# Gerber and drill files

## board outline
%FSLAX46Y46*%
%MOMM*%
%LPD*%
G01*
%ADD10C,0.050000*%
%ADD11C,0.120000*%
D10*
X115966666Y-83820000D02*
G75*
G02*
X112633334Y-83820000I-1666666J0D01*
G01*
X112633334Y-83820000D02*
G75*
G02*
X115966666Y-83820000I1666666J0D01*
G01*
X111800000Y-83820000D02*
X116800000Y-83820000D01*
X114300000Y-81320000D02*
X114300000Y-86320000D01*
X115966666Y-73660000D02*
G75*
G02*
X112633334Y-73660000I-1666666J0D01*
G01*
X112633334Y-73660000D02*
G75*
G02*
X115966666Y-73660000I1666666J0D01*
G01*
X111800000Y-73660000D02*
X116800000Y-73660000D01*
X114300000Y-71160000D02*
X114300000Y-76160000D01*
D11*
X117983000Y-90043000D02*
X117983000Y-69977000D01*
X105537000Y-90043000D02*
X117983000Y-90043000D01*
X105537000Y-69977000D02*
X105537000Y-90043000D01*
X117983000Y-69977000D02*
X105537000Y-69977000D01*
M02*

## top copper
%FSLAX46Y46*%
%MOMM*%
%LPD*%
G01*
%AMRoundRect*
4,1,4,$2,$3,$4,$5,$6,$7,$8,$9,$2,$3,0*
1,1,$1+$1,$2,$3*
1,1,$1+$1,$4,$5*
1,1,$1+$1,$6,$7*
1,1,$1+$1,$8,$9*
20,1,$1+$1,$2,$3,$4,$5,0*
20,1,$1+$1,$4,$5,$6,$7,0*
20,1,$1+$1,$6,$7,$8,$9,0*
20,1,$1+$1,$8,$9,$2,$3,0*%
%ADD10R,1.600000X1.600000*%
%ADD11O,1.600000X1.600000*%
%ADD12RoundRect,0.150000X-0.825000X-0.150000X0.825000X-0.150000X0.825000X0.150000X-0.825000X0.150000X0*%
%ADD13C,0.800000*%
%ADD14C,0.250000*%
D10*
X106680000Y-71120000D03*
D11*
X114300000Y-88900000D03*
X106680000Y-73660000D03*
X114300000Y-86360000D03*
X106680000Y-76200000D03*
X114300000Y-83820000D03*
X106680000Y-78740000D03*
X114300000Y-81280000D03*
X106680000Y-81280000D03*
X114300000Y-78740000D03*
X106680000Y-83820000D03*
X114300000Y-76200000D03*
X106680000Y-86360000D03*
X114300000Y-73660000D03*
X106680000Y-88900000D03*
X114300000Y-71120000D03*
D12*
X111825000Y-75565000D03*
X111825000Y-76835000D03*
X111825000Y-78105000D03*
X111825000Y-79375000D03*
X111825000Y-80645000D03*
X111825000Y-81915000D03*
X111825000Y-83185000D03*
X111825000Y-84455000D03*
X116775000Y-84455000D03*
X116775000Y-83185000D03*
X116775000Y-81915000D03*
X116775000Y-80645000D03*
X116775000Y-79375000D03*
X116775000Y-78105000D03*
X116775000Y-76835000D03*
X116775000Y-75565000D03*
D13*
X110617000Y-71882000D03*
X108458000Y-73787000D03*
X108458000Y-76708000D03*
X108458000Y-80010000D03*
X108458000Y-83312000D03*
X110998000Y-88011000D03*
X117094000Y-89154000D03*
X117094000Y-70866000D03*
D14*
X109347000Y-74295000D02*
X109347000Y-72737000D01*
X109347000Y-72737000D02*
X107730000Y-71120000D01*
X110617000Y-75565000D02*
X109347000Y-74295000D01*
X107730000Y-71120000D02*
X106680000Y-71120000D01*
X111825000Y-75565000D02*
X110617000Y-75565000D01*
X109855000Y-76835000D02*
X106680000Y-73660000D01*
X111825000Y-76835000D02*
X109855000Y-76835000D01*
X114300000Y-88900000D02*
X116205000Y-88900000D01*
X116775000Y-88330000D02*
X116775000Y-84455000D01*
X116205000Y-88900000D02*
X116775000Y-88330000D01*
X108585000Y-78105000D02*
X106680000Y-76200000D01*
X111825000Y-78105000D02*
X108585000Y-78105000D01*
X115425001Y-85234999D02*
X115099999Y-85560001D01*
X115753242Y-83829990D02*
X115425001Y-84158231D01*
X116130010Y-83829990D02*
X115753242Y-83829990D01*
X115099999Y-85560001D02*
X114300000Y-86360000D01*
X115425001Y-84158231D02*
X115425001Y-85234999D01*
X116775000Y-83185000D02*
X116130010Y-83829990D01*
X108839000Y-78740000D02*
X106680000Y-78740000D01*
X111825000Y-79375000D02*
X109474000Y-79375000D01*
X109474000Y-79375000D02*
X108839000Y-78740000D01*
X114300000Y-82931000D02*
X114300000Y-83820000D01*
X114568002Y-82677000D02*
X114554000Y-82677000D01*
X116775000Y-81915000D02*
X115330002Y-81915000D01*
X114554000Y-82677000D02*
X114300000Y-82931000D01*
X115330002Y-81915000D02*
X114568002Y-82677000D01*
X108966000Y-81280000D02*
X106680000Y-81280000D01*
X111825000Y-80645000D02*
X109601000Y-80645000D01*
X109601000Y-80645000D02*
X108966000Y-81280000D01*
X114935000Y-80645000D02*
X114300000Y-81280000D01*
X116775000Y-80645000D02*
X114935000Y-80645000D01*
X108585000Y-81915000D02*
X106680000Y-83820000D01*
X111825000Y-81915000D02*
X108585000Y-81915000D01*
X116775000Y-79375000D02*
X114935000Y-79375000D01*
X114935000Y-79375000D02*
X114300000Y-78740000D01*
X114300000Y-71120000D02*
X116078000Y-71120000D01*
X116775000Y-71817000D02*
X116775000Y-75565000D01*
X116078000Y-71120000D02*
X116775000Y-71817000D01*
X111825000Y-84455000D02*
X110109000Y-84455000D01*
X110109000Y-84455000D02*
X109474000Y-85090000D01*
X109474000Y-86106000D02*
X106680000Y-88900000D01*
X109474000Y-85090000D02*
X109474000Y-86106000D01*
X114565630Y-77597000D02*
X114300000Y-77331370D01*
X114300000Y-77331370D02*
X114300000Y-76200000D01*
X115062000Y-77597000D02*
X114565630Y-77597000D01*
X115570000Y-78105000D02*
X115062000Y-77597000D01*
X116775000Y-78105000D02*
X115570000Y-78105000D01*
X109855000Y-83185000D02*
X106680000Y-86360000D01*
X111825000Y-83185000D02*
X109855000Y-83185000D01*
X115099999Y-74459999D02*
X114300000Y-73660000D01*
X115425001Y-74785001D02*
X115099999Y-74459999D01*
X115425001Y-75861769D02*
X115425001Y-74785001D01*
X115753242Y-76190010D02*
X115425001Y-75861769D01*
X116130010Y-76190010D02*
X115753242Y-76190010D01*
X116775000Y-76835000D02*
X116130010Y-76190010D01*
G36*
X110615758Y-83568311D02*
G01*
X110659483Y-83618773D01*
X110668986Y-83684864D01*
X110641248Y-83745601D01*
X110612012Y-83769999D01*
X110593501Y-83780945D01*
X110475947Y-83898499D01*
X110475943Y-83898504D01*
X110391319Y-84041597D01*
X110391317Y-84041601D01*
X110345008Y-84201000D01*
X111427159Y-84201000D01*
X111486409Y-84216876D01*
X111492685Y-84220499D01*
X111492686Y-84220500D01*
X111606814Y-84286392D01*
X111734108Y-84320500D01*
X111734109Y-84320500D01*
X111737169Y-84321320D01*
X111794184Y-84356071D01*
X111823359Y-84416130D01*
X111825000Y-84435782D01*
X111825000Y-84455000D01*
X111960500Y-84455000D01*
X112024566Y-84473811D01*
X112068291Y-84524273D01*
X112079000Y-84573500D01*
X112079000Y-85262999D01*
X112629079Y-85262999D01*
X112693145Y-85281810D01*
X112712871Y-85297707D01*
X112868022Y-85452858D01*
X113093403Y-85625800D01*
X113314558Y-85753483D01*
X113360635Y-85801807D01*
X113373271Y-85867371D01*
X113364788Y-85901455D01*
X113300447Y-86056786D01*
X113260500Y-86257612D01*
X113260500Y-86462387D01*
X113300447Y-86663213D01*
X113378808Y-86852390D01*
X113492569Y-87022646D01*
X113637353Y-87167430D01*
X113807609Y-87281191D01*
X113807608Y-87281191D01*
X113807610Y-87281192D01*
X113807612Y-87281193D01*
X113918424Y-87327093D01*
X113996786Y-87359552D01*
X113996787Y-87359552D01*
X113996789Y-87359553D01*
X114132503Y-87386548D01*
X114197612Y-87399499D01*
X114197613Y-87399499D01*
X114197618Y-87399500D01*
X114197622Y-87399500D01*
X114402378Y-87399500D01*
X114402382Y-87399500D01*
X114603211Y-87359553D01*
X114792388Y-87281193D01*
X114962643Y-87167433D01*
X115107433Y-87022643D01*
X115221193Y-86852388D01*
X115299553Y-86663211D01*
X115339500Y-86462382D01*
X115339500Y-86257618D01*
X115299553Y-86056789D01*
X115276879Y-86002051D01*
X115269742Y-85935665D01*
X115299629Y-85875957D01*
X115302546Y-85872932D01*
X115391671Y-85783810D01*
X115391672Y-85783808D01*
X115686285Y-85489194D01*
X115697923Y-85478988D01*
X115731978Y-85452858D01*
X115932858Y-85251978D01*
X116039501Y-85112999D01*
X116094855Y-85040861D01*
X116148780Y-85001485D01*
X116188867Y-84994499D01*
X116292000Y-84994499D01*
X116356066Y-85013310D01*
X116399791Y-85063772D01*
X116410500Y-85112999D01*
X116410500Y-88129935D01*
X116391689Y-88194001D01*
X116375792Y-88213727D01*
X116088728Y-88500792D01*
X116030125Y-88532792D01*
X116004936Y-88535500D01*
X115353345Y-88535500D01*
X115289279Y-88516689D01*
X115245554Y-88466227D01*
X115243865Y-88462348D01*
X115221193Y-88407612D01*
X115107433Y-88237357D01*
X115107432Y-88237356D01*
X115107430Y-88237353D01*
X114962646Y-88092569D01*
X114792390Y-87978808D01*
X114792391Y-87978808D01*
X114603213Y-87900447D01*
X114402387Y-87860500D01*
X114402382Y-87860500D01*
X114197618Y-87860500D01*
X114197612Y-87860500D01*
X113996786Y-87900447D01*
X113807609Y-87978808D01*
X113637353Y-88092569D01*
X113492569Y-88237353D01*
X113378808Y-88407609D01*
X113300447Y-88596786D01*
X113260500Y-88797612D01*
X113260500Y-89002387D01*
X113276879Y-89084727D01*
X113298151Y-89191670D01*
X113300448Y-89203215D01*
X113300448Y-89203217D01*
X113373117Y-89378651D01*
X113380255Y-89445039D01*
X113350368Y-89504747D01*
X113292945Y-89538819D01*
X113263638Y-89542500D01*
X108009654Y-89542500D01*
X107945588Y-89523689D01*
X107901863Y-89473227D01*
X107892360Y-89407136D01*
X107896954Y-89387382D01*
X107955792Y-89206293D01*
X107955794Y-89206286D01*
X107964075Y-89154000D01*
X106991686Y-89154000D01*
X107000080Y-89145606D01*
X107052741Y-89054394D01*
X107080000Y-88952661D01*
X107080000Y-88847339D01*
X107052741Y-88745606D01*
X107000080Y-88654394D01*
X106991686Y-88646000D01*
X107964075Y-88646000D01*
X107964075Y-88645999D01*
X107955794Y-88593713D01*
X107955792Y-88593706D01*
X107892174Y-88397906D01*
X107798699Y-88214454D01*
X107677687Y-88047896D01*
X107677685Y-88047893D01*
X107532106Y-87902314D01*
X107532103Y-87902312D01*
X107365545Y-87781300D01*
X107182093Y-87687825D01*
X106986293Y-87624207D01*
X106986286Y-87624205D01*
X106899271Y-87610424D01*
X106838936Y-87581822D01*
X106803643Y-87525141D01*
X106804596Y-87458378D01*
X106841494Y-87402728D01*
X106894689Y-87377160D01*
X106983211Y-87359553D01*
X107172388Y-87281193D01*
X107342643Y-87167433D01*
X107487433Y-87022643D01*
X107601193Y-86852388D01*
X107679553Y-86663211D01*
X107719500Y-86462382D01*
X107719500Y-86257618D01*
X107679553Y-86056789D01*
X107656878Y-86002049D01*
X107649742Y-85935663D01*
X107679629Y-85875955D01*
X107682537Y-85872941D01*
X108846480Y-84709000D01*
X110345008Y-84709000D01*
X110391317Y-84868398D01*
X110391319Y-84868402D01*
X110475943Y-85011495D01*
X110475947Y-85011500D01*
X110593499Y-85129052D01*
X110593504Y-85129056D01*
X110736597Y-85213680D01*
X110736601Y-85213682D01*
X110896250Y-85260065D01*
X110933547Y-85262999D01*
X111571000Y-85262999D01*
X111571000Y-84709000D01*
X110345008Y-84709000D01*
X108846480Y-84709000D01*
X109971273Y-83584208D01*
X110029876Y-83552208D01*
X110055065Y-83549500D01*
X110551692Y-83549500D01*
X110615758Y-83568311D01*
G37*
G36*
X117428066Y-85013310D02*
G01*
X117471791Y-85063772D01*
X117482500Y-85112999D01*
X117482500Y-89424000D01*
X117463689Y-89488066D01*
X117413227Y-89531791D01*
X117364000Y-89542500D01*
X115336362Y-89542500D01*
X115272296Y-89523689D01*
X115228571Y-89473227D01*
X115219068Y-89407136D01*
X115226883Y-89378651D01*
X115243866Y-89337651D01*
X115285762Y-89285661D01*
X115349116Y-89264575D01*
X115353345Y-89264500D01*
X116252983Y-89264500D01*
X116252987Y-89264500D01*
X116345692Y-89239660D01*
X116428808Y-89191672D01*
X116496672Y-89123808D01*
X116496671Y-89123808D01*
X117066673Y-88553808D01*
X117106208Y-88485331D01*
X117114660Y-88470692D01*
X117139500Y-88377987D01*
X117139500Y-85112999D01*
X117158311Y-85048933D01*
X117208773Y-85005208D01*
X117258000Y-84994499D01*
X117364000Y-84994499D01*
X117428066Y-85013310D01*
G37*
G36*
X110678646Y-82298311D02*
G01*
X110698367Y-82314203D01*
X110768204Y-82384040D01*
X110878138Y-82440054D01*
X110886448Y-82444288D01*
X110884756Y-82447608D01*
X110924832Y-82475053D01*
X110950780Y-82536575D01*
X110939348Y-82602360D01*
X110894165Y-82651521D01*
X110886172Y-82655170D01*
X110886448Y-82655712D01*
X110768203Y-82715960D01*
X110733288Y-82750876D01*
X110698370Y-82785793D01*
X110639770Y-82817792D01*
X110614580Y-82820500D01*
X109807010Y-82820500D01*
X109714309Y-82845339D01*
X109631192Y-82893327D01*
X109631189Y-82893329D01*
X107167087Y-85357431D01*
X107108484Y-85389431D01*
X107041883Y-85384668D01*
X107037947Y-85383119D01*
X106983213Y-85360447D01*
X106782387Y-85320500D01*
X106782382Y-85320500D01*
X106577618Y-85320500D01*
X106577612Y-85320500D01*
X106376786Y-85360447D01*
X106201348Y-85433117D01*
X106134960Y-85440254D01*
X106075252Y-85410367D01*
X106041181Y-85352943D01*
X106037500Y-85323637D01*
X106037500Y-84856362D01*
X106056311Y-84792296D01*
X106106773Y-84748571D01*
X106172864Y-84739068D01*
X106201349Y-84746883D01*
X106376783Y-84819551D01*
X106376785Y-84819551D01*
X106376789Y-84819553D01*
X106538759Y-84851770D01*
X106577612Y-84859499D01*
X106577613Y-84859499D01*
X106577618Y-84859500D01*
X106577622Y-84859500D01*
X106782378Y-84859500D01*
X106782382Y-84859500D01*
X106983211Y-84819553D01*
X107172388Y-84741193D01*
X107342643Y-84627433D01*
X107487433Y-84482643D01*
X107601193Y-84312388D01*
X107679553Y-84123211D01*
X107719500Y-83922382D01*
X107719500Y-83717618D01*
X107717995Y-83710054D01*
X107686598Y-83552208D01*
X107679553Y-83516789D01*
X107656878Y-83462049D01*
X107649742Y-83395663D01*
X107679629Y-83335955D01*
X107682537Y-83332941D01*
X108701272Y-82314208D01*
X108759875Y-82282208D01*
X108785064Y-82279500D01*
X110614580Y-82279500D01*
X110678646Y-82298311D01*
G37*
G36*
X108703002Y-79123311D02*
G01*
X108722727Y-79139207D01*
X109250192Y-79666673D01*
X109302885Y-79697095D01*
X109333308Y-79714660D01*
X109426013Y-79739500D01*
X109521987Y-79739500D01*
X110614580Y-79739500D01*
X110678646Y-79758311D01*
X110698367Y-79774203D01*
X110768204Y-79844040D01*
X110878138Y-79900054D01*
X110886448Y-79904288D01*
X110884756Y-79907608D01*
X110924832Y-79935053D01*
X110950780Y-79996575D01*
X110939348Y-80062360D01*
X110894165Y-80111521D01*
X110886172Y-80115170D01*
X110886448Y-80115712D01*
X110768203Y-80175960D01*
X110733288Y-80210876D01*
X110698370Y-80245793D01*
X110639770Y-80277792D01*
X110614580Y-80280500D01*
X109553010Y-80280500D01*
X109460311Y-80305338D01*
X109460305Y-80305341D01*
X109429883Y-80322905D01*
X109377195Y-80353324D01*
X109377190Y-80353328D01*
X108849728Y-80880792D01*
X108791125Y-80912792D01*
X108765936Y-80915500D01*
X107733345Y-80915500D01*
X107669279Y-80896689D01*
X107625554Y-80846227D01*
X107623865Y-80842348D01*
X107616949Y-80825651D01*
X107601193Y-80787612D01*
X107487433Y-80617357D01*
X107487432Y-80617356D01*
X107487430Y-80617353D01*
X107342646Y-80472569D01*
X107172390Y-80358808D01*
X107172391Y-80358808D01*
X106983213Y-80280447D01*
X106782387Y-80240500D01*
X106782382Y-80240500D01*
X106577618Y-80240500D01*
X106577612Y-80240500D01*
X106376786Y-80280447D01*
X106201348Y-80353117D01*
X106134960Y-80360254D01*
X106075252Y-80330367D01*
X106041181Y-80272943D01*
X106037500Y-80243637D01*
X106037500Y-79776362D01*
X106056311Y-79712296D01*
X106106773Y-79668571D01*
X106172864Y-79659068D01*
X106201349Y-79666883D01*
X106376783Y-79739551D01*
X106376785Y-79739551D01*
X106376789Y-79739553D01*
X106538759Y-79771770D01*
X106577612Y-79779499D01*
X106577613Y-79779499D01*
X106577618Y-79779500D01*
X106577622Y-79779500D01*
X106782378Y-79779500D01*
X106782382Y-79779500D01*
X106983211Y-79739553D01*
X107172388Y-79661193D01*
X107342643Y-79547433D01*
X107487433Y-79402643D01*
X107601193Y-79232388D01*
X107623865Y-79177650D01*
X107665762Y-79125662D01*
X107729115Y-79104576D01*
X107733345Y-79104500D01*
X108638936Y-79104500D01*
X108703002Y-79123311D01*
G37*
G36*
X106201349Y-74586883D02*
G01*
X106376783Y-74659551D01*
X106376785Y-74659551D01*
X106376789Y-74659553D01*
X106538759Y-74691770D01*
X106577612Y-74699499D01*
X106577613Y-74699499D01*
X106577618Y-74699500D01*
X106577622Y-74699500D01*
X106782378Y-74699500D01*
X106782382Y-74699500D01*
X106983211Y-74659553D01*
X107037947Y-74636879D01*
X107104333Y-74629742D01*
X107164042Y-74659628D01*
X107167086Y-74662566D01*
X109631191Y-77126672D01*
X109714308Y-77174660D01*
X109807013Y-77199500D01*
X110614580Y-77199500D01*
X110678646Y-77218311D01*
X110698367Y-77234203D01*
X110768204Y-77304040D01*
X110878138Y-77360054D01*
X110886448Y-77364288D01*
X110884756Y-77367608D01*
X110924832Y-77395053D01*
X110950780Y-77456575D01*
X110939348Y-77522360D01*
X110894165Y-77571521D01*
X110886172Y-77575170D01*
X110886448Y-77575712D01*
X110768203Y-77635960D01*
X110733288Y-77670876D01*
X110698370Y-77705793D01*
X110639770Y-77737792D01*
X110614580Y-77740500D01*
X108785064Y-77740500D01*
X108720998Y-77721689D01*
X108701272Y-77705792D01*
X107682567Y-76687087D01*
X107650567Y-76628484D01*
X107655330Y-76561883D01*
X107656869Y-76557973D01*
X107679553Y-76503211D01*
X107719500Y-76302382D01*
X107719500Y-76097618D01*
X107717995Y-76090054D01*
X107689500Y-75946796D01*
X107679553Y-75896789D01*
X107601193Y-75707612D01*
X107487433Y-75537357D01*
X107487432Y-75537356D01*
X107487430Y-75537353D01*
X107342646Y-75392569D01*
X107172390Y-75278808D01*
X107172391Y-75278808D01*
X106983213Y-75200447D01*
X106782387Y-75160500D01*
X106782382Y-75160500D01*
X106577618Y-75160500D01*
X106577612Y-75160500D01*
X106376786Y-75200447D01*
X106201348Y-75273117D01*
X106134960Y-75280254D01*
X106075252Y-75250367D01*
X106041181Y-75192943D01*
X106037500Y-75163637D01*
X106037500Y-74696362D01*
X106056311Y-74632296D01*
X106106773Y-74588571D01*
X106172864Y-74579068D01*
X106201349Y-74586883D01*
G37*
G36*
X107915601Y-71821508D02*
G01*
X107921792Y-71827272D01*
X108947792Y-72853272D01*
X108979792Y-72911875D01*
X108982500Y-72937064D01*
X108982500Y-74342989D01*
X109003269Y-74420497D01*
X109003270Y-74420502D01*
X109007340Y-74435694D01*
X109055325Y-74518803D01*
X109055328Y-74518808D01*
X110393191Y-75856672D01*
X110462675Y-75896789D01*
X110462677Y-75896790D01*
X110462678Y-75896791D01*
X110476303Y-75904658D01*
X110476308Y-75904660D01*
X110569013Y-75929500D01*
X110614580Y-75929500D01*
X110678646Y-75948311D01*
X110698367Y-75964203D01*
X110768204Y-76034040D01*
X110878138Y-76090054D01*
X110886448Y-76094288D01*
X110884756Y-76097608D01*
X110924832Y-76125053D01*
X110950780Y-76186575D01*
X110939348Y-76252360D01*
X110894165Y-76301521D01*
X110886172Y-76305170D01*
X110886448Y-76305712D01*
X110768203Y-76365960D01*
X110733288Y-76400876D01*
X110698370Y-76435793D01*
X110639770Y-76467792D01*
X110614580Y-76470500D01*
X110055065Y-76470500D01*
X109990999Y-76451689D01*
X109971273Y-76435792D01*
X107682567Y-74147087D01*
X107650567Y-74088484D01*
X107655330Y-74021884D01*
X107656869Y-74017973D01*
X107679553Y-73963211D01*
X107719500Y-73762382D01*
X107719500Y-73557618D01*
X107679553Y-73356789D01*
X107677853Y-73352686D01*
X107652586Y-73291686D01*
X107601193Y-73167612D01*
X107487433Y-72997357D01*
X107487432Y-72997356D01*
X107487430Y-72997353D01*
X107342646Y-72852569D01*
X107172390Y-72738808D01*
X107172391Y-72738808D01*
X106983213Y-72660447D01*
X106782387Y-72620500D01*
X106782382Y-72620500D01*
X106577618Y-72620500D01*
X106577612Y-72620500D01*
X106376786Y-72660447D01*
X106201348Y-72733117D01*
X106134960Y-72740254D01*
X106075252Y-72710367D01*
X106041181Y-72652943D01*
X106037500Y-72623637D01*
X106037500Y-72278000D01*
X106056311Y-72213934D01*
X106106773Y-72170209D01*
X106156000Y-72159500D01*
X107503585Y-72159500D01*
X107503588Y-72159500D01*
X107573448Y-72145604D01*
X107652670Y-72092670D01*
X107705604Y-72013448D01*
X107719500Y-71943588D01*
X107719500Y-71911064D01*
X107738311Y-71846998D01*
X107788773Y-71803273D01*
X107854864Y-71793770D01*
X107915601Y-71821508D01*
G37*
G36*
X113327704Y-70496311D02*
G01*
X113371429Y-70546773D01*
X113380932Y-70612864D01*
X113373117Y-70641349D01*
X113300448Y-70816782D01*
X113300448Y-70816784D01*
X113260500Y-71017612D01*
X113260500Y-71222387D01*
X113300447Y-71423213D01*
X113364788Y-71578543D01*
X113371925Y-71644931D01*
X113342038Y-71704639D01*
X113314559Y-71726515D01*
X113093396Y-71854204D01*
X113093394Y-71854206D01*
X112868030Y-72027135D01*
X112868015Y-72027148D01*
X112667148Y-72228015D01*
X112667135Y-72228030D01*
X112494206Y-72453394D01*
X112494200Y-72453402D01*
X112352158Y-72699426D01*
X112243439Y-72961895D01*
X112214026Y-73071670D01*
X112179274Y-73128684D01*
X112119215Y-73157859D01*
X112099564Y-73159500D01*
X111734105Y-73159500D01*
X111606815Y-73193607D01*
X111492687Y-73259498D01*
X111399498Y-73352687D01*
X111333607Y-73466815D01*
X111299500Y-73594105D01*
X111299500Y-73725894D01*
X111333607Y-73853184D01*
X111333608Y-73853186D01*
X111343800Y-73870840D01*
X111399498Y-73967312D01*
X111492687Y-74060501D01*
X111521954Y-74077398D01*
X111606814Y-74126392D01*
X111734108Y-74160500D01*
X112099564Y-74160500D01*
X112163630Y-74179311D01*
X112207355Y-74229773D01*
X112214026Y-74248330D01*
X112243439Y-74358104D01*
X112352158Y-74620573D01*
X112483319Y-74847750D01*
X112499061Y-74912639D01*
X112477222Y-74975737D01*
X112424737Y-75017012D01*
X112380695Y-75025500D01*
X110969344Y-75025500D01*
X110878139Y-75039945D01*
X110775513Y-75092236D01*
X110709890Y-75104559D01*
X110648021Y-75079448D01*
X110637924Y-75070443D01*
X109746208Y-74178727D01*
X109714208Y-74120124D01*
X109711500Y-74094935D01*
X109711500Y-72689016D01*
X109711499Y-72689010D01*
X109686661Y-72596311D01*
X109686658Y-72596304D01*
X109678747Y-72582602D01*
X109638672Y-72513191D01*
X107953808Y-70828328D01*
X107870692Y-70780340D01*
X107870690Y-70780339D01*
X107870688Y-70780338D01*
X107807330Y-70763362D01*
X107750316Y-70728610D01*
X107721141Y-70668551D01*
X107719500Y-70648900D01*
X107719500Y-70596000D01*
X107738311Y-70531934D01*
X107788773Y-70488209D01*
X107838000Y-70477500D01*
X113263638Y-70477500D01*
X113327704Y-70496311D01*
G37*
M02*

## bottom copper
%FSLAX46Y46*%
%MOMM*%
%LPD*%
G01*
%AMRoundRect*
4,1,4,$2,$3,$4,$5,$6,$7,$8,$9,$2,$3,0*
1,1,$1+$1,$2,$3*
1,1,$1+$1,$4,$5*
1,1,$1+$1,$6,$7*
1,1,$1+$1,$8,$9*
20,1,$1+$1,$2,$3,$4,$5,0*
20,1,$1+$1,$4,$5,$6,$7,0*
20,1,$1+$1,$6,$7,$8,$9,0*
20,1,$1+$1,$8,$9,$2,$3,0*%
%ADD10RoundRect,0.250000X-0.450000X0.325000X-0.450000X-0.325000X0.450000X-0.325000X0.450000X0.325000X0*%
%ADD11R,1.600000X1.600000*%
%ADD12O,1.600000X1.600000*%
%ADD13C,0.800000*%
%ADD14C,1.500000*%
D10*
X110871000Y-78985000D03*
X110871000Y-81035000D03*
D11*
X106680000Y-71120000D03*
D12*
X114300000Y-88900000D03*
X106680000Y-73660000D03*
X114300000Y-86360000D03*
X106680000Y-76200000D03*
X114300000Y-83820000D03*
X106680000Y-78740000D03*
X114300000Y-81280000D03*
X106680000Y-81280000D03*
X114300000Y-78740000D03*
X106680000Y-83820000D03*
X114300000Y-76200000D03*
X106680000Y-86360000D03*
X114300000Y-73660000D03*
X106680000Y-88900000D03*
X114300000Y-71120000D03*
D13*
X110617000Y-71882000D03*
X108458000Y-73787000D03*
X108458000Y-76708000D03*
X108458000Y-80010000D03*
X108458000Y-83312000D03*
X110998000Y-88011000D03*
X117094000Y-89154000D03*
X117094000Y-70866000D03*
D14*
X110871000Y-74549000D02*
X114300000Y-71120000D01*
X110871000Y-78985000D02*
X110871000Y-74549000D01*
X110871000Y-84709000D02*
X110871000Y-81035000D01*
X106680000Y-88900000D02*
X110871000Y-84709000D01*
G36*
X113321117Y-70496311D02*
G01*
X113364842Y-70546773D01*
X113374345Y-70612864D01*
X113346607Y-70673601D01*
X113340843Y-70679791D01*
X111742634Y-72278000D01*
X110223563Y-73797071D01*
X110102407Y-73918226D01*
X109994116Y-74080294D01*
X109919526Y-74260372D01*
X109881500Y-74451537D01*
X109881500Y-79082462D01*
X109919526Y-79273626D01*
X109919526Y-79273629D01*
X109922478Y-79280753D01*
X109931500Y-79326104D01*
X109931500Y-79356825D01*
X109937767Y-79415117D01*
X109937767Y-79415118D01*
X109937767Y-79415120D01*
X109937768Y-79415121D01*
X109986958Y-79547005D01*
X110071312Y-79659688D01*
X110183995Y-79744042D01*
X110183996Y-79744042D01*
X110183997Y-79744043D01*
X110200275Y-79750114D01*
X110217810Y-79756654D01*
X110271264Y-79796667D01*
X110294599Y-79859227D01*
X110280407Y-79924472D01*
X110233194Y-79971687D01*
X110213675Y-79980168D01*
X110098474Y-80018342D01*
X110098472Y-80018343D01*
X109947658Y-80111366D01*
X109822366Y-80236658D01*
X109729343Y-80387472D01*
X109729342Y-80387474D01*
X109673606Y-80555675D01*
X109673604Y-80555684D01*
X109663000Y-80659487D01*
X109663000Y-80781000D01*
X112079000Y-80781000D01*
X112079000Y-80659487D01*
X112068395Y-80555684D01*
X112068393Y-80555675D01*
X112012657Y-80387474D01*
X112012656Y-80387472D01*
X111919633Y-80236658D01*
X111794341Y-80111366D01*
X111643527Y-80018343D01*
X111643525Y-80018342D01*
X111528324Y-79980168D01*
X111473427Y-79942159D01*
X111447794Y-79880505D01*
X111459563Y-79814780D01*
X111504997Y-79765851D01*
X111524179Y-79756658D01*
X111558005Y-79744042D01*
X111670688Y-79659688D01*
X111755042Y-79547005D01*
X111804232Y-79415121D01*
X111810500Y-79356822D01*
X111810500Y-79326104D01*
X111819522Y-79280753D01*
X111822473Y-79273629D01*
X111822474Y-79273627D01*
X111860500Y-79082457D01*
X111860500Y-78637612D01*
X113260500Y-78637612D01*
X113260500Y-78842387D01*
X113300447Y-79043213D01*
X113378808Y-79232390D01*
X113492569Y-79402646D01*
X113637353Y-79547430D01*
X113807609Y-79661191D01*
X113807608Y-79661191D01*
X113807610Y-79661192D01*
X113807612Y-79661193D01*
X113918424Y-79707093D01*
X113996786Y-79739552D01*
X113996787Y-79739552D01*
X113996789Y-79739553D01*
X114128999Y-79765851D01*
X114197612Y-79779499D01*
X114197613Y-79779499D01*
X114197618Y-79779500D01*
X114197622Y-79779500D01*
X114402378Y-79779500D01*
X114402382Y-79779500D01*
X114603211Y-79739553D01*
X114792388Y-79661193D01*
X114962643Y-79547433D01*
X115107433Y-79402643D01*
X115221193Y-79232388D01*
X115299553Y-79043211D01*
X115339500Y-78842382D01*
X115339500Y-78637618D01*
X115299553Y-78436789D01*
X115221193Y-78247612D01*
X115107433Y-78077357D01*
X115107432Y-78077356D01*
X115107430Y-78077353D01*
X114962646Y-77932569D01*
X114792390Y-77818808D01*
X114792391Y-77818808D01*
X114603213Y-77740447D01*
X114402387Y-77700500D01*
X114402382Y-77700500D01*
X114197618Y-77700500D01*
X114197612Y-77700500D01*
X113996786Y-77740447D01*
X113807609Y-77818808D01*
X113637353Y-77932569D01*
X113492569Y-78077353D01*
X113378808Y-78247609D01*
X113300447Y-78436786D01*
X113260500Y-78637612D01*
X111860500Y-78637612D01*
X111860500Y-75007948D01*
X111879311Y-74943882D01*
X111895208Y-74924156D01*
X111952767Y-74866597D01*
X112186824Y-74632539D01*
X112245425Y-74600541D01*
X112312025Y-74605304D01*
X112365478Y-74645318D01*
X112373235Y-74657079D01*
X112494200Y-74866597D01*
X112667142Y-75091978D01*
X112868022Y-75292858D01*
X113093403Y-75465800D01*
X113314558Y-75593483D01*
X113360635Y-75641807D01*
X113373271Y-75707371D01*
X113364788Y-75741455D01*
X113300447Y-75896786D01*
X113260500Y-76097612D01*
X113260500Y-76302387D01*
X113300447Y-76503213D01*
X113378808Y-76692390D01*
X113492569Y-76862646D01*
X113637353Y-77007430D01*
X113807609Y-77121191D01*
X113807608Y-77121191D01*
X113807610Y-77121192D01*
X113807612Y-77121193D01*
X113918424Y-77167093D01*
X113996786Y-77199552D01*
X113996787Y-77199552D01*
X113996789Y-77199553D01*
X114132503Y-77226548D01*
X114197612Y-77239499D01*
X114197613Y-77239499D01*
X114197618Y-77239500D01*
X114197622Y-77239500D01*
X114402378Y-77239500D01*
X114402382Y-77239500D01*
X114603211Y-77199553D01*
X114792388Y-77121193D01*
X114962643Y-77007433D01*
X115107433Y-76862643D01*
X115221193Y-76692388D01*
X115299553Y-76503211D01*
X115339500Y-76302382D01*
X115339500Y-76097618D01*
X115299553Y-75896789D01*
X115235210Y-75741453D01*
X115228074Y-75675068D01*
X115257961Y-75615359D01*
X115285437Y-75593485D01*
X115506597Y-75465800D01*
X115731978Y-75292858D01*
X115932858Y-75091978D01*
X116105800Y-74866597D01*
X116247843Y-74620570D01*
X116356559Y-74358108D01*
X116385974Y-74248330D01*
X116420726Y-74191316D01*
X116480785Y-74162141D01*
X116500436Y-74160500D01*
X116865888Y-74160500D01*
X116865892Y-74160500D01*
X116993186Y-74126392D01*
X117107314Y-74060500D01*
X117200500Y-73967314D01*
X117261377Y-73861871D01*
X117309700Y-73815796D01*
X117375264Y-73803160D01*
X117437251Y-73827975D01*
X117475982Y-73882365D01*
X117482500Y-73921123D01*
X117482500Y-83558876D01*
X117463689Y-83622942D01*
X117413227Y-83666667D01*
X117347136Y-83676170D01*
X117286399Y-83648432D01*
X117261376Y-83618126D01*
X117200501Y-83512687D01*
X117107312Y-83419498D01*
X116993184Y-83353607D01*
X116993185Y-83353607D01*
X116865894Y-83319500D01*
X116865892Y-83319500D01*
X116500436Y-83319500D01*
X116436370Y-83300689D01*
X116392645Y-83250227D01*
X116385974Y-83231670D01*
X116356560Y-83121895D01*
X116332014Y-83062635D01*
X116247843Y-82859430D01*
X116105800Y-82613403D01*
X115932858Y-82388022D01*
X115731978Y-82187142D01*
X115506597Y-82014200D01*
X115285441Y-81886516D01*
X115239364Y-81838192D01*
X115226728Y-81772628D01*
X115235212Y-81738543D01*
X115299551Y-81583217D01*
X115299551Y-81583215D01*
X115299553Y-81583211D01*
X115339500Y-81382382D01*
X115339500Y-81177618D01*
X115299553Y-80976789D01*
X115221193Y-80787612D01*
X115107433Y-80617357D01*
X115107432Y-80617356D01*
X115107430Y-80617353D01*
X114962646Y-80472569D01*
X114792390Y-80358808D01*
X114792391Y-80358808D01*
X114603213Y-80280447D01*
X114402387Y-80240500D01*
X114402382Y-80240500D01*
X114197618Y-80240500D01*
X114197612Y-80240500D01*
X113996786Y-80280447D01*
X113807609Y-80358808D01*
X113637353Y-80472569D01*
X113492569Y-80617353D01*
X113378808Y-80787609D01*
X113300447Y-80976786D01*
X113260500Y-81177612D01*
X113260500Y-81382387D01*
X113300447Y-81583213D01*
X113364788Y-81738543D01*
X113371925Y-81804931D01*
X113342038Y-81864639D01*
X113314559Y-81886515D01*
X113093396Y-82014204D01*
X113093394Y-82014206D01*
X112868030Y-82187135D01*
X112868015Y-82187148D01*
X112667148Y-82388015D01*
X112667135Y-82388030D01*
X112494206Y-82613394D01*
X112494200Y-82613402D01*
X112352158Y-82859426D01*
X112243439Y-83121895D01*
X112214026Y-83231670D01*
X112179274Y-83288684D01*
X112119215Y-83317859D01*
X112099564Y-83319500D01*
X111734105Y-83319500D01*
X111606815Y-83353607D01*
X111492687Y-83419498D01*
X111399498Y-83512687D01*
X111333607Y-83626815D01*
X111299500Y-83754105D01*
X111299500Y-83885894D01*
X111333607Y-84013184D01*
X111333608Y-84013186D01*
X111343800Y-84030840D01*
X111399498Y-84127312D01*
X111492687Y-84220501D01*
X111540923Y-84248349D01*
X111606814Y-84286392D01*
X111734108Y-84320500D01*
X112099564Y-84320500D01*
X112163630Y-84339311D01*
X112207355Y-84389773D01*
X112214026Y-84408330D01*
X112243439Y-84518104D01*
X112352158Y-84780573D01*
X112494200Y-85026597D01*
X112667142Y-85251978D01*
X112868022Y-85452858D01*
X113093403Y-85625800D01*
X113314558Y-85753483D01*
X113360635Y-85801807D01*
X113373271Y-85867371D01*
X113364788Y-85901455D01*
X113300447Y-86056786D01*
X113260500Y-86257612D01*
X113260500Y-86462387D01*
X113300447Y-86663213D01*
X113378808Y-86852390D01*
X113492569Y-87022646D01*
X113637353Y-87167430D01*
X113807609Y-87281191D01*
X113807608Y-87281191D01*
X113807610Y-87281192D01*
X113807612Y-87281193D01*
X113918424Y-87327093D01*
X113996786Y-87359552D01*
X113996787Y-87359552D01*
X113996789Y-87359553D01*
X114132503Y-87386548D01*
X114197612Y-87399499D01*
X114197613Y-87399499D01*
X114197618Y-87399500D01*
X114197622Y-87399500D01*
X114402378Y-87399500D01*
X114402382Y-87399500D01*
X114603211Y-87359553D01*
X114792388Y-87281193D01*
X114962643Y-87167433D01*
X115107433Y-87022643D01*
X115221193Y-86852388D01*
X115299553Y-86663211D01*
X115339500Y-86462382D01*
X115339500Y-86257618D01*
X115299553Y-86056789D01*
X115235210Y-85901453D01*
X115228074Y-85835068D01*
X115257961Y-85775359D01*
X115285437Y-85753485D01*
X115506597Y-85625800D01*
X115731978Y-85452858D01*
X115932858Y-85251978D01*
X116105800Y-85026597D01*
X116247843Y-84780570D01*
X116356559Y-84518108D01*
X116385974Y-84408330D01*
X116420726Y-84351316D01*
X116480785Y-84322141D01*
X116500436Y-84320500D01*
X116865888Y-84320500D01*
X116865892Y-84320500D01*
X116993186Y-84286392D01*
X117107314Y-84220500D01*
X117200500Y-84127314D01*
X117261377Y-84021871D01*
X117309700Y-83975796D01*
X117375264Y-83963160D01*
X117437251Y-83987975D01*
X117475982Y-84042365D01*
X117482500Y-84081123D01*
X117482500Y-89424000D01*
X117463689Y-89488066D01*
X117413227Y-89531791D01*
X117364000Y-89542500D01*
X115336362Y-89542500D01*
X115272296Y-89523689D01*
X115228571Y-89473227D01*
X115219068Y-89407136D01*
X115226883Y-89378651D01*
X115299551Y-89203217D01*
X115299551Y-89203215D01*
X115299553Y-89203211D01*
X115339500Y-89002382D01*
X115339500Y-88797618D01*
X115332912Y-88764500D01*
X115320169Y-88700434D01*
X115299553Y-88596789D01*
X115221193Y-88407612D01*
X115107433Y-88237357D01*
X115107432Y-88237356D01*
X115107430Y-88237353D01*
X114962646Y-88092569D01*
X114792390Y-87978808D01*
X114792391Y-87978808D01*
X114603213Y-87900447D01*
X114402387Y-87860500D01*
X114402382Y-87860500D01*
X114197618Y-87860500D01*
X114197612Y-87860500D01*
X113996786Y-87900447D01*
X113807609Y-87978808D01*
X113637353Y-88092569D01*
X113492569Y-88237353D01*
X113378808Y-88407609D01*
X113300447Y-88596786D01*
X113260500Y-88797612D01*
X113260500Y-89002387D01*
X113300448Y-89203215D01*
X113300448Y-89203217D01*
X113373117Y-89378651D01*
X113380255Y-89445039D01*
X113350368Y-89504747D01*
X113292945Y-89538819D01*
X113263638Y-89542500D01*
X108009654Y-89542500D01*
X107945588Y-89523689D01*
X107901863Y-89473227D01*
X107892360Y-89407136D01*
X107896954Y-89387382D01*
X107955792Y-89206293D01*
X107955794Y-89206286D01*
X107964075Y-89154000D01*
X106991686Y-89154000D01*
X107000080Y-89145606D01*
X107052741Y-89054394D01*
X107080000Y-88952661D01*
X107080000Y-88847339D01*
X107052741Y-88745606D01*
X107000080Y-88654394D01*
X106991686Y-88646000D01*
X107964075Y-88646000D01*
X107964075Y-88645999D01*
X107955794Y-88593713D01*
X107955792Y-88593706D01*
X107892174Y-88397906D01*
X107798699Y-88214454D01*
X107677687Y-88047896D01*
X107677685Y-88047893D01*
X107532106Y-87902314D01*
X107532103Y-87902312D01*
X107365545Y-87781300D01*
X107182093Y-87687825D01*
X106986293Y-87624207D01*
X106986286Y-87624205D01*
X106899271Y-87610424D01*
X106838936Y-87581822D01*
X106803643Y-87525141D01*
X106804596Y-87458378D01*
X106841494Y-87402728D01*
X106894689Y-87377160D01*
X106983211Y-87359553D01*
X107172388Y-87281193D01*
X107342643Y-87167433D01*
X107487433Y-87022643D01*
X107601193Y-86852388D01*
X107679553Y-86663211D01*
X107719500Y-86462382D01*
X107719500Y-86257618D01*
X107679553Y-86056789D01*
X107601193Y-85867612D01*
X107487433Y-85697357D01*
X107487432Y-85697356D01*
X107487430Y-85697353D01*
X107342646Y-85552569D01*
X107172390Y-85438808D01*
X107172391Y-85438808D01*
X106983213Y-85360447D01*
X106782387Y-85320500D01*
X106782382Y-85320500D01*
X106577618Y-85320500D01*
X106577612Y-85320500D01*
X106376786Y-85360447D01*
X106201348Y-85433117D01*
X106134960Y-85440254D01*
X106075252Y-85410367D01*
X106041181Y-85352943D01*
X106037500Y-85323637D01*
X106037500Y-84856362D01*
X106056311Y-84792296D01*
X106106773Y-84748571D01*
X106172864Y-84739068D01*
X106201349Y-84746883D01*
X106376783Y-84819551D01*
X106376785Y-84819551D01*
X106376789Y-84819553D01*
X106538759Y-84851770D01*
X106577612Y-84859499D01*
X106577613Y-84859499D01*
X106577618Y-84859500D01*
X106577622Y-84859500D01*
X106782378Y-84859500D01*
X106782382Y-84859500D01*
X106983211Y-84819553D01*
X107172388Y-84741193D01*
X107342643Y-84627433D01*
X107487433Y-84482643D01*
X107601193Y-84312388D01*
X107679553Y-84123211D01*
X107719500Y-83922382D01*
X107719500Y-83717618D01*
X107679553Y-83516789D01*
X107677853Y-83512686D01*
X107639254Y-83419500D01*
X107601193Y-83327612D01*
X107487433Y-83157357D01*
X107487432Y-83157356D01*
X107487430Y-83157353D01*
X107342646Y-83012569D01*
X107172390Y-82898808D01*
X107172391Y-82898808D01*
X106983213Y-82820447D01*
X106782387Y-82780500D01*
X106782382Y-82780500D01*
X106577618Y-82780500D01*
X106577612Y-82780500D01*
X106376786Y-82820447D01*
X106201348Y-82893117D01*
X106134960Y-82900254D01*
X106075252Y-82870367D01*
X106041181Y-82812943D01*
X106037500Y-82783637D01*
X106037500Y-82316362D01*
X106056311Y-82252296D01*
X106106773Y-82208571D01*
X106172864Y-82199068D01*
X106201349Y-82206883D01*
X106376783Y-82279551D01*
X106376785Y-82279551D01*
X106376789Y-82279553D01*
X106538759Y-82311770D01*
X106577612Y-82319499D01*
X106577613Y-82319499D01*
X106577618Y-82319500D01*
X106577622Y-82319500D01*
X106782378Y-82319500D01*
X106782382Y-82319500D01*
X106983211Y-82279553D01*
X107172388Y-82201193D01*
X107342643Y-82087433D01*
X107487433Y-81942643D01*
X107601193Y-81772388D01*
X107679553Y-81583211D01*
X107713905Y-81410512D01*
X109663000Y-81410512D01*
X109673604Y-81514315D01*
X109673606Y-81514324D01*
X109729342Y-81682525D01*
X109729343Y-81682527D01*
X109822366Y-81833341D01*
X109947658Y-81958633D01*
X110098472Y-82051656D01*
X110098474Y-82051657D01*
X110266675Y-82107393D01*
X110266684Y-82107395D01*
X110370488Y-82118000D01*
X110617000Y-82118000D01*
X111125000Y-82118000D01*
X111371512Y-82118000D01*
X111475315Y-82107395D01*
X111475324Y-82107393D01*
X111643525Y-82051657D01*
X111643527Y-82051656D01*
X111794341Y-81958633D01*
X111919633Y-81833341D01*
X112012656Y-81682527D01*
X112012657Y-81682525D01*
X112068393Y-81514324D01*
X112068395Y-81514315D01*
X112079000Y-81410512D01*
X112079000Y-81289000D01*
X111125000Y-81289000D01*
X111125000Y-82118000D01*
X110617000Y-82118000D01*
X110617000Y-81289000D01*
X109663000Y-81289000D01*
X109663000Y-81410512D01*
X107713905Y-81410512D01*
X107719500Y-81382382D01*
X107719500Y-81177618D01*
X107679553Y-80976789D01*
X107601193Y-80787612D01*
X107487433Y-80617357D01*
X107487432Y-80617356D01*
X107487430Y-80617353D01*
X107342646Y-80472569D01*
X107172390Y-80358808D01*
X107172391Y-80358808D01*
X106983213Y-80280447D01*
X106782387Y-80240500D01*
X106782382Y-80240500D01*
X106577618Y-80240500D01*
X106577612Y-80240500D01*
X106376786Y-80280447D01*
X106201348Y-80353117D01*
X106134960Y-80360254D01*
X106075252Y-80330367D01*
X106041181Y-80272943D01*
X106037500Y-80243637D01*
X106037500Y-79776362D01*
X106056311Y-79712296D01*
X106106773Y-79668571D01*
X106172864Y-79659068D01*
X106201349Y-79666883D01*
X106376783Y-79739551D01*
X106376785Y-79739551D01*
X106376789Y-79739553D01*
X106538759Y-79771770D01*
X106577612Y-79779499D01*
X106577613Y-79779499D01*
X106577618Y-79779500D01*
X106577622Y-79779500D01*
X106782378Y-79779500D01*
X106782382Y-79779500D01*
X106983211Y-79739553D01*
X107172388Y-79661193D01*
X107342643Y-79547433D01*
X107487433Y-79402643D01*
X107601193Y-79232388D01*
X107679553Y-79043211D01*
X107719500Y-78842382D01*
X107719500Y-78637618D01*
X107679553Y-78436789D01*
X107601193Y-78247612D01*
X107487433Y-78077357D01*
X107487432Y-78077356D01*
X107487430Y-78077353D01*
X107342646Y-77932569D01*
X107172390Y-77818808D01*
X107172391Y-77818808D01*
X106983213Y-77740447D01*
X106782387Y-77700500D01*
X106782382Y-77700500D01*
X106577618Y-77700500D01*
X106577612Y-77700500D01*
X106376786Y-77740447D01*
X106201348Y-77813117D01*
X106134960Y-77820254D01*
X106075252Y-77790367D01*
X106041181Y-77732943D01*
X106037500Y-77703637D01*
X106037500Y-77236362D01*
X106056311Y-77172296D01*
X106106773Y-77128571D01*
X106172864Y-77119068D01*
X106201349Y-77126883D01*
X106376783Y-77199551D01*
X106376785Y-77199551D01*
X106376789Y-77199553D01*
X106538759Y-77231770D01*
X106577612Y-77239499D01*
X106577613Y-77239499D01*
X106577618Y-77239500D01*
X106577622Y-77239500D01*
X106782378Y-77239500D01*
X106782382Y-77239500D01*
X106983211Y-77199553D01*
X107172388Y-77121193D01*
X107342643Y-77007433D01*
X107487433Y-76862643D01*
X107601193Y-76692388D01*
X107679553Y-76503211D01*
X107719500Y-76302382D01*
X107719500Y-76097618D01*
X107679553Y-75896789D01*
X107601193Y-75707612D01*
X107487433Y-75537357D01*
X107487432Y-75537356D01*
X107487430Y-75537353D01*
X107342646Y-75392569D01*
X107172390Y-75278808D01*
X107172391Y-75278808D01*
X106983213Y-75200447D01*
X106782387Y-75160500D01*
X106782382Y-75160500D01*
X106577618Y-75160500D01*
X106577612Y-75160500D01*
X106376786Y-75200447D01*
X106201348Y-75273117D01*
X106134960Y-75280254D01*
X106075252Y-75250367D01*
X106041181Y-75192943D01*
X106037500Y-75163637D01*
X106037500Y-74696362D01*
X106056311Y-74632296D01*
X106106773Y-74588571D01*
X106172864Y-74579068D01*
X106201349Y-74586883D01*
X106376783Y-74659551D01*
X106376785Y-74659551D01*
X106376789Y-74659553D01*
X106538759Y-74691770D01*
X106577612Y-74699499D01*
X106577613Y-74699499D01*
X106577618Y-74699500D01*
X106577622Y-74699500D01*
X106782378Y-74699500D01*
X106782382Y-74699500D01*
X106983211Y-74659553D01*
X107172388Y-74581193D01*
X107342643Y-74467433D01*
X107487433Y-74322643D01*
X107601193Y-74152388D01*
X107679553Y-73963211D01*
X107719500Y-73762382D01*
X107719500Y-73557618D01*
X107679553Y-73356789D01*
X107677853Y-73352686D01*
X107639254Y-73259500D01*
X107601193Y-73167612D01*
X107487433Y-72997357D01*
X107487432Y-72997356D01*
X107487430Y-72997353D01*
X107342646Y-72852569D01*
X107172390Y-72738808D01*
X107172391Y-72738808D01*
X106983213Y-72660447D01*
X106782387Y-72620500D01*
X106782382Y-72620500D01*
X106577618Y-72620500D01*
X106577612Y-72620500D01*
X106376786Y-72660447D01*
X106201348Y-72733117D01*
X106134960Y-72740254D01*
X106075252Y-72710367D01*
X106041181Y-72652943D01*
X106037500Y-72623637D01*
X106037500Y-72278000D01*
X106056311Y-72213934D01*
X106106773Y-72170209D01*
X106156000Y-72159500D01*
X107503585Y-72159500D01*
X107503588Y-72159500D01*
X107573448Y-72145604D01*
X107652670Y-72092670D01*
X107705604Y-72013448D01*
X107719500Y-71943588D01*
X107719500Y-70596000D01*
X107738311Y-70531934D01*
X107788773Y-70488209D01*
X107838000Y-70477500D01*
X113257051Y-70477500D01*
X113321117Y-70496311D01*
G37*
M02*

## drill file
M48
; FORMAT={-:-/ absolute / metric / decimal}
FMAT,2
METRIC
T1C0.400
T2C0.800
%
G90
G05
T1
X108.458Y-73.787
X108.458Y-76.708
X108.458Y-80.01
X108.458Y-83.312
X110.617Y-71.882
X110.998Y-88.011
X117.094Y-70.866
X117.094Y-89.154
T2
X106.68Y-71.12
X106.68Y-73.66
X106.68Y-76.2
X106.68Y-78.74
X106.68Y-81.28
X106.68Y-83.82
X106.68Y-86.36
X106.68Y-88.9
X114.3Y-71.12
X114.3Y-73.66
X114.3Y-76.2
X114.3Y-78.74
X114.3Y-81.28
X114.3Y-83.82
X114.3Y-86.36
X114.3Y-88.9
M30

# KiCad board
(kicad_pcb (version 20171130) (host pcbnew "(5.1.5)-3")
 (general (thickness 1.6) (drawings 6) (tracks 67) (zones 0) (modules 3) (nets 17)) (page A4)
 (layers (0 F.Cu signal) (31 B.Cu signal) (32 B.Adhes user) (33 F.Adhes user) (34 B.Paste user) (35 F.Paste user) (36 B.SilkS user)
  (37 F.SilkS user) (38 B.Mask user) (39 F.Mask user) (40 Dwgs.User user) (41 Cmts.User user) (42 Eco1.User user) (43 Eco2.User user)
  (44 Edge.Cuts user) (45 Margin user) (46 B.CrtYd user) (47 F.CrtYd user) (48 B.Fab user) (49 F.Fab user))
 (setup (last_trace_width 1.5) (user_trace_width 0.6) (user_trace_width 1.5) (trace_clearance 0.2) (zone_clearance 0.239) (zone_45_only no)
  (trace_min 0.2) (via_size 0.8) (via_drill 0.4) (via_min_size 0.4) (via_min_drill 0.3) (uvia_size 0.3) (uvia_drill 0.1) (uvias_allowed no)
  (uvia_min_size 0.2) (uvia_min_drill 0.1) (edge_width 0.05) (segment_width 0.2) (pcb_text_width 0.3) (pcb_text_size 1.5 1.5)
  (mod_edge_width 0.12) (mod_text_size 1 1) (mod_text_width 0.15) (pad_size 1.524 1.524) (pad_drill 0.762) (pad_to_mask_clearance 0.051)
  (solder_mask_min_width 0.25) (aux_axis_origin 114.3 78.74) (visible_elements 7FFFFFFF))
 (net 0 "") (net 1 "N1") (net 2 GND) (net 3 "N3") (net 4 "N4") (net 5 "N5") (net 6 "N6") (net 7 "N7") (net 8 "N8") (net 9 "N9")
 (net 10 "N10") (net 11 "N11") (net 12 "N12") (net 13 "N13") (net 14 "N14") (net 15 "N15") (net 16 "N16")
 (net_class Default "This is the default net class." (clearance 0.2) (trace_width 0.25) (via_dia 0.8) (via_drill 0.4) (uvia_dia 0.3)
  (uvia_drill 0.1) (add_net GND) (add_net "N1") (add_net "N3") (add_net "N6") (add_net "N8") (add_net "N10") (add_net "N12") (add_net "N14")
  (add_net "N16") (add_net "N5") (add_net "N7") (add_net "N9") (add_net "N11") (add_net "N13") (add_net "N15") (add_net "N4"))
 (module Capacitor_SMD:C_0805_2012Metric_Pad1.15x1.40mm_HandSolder (layer B.Cu) (at 110.871 80.01 270)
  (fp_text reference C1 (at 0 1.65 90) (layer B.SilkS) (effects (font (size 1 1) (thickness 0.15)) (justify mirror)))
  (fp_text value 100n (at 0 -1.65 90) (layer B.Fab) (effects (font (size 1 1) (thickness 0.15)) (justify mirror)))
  (pad 1 smd roundrect (at -1.025 0 270) (size 1.15 1.4) (layers B.Cu B.Paste B.Mask) (roundrect_rratio 0.217391) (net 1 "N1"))
  (pad 2 smd roundrect (at 1.025 0 270) (size 1.15 1.4) (layers B.Cu B.Paste B.Mask) (roundrect_rratio 0.217391) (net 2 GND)))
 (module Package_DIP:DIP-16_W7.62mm (layer F.Cu) (at 106.68 71.12)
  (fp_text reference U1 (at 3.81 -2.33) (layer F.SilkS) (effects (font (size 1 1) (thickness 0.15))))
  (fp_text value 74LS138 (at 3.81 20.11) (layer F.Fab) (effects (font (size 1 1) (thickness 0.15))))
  (pad 1 thru_hole rect (at 0 0) (size 1.6 1.6) (drill 0.8) (layers *.Cu *.Mask) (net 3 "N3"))
  (pad 9 thru_hole oval (at 7.62 17.78) (size 1.6 1.6) (drill 0.8) (layers *.Cu *.Mask) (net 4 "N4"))
  (pad 2 thru_hole oval (at 0 2.54) (size 1.6 1.6) (drill 0.8) (layers *.Cu *.Mask) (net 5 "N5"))
  (pad 10 thru_hole oval (at 7.62 15.24) (size 1.6 1.6) (drill 0.8) (layers *.Cu *.Mask) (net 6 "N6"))
  (pad 3 thru_hole oval (at 0 5.08) (size 1.6 1.6) (drill 0.8) (layers *.Cu *.Mask) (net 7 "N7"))
  (pad 11 thru_hole oval (at 7.62 12.7) (size 1.6 1.6) (drill 0.8) (layers *.Cu *.Mask) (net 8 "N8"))
  (pad 4 thru_hole oval (at 0 7.62) (size 1.6 1.6) (drill 0.8) (layers *.Cu *.Mask) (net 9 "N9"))
  (pad 12 thru_hole oval (at 7.62 10.16) (size 1.6 1.6) (drill 0.8) (layers *.Cu *.Mask) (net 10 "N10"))
  (pad 5 thru_hole oval (at 0 10.16) (size 1.6 1.6) (drill 0.8) (layers *.Cu *.Mask) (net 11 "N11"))
  (pad 13 thru_hole oval (at 7.62 7.62) (size 1.6 1.6) (drill 0.8) (layers *.Cu *.Mask) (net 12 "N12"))
  (pad 6 thru_hole oval (at 0 12.7) (size 1.6 1.6) (drill 0.8) (layers *.Cu *.Mask) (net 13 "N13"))
  (pad 14 thru_hole oval (at 7.62 5.08) (size 1.6 1.6) (drill 0.8) (layers *.Cu *.Mask) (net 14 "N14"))
  (pad 7 thru_hole oval (at 0 15.24) (size 1.6 1.6) (drill 0.8) (layers *.Cu *.Mask) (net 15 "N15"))
  (pad 15 thru_hole oval (at 7.62 2.54) (size 1.6 1.6) (drill 0.8) (layers *.Cu *.Mask) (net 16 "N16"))
  (pad 8 thru_hole oval (at 0 17.78) (size 1.6 1.6) (drill 0.8) (layers *.Cu *.Mask) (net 2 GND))
  (pad 16 thru_hole oval (at 7.62 0) (size 1.6 1.6) (drill 0.8) (layers *.Cu *.Mask) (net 1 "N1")))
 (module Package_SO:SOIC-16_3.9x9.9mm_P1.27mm (layer F.Cu) (at 114.3 80.01)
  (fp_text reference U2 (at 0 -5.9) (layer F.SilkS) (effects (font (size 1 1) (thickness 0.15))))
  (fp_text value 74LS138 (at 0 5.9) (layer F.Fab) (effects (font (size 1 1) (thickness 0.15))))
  (pad 1 smd roundrect (at -2.475 -4.445) (size 1.95 0.6) (layers F.Cu F.Paste F.Mask) (roundrect_rratio 0.25) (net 3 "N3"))
  (pad 2 smd roundrect (at -2.475 -3.175) (size 1.95 0.6) (layers F.Cu F.Paste F.Mask) (roundrect_rratio 0.25) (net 5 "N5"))
  (pad 3 smd roundrect (at -2.475 -1.905) (size 1.95 0.6) (layers F.Cu F.Paste F.Mask) (roundrect_rratio 0.25) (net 7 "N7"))
  (pad 4 smd roundrect (at -2.475 -0.635) (size 1.95 0.6) (layers F.Cu F.Paste F.Mask) (roundrect_rratio 0.25) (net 9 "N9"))
  (pad 5 smd roundrect (at -2.475 0.635) (size 1.95 0.6) (layers F.Cu F.Paste F.Mask) (roundrect_rratio 0.25) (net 11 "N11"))
  (pad 6 smd roundrect (at -2.475 1.905) (size 1.95 0.6) (layers F.Cu F.Paste F.Mask) (roundrect_rratio 0.25) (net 13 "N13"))
  (pad 7 smd roundrect (at -2.475 3.175) (size 1.95 0.6) (layers F.Cu F.Paste F.Mask) (roundrect_rratio 0.25) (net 15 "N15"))
  (pad 8 smd roundrect (at -2.475 4.445) (size 1.95 0.6) (layers F.Cu F.Paste F.Mask) (roundrect_rratio 0.25) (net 2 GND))
  (pad 9 smd roundrect (at 2.475 4.445) (size 1.95 0.6) (layers F.Cu F.Paste F.Mask) (roundrect_rratio 0.25) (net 4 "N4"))
  (pad 10 smd roundrect (at 2.475 3.175) (size 1.95 0.6) (layers F.Cu F.Paste F.Mask) (roundrect_rratio 0.25) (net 6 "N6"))
  (pad 11 smd roundrect (at 2.475 1.905) (size 1.95 0.6) (layers F.Cu F.Paste F.Mask) (roundrect_rratio 0.25) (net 8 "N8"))
  (pad 12 smd roundrect (at 2.475 0.635) (size 1.95 0.6) (layers F.Cu F.Paste F.Mask) (roundrect_rratio 0.25) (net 10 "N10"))
  (pad 13 smd roundrect (at 2.475 -0.635) (size 1.95 0.6) (layers F.Cu F.Paste F.Mask) (roundrect_rratio 0.25) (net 12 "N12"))
  (pad 14 smd roundrect (at 2.475 -1.905) (size 1.95 0.6) (layers F.Cu F.Paste F.Mask) (roundrect_rratio 0.25) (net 14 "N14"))
  (pad 15 smd roundrect (at 2.475 -3.175) (size 1.95 0.6) (layers F.Cu F.Paste F.Mask) (roundrect_rratio 0.25) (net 16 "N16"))
  (pad 16 smd roundrect (at 2.475 -4.445) (size 1.95 0.6) (layers F.Cu F.Paste F.Mask) (roundrect_rratio 0.25) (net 1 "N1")))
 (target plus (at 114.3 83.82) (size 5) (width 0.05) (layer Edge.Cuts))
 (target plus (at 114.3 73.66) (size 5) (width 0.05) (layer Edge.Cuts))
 (gr_line (start 117.983 90.043) (end 117.983 69.977) (layer Edge.Cuts) (width 0.12))
 (gr_line (start 105.537 90.043) (end 117.983 90.043) (layer Edge.Cuts) (width 0.12))
 (gr_line (start 105.537 69.977) (end 105.537 90.043) (layer Edge.Cuts) (width 0.12))
 (gr_line (start 117.983 69.977) (end 105.537 69.977) (layer Edge.Cuts) (width 0.12))
 (segment (start 109.347 74.295) (end 109.347 72.737) (width 0.25) (layer F.Cu) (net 3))
 (segment (start 109.347 72.737) (end 107.73 71.12) (width 0.25) (layer F.Cu) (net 3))
 (segment (start 110.617 75.565) (end 109.347 74.295) (width 0.25) (layer F.Cu) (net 3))
 (segment (start 107.73 71.12) (end 106.68 71.12) (width 0.25) (layer F.Cu) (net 3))
 (segment (start 111.825 75.565) (end 110.617 75.565) (width 0.25) (layer F.Cu) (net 3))
 (segment (start 109.855 76.835) (end 106.68 73.66) (width 0.25) (layer F.Cu) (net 5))
 (segment (start 111.825 76.835) (end 109.855 76.835) (width 0.25) (layer F.Cu) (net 5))
 (segment (start 114.3 88.9) (end 116.205 88.9) (width 0.25) (layer F.Cu) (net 4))
 (segment (start 116.775 88.33) (end 116.775 84.455) (width 0.25) (layer F.Cu) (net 4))
 (segment (start 116.205 88.9) (end 116.775 88.33) (width 0.25) (layer F.Cu) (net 4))
 (segment (start 108.585 78.105) (end 106.68 76.2) (width 0.25) (layer F.Cu) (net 7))
 (segment (start 111.825 78.105) (end 108.585 78.105) (width 0.25) (layer F.Cu) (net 7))
 (segment (start 115.425001 85.234999) (end 115.099999 85.560001) (width 0.25) (layer F.Cu) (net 6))
 (segment (start 115.753242 83.82999) (end 115.425001 84.158231) (width 0.25) (layer F.Cu) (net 6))
 (segment (start 116.13001 83.82999) (end 115.753242 83.82999) (width 0.25) (layer F.Cu) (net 6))
 (segment (start 115.099999 85.560001) (end 114.3 86.36) (width 0.25) (layer F.Cu) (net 6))
 (segment (start 115.425001 84.158231) (end 115.425001 85.234999) (width 0.25) (layer F.Cu) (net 6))
 (segment (start 116.775 83.185) (end 116.13001 83.82999) (width 0.25) (layer F.Cu) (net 6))
 (segment (start 108.839 78.74) (end 106.68 78.74) (width 0.25) (layer F.Cu) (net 9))
 (segment (start 111.825 79.375) (end 109.474 79.375) (width 0.25) (layer F.Cu) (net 9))
 (segment (start 109.474 79.375) (end 108.839 78.74) (width 0.25) (layer F.Cu) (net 9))
 (segment (start 114.3 82.931) (end 114.3 83.82) (width 0.25) (layer F.Cu) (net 8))
 (segment (start 114.568002 82.677) (end 114.554 82.677) (width 0.25) (layer F.Cu) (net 8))
 (segment (start 116.775 81.915) (end 115.330002 81.915) (width 0.25) (layer F.Cu) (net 8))
 (segment (start 114.554 82.677) (end 114.3 82.931) (width 0.25) (layer F.Cu) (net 8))
 (segment (start 115.330002 81.915) (end 114.568002 82.677) (width 0.25) (layer F.Cu) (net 8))
 (segment (start 108.966 81.28) (end 106.68 81.28) (width 0.25) (layer F.Cu) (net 11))
 (segment (start 111.825 80.645) (end 109.601 80.645) (width 0.25) (layer F.Cu) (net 11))
 (segment (start 109.601 80.645) (end 108.966 81.28) (width 0.25) (layer F.Cu) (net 11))
 (segment (start 114.935 80.645) (end 114.3 81.28) (width 0.25) (layer F.Cu) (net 10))
 (segment (start 116.775 80.645) (end 114.935 80.645) (width 0.25) (layer F.Cu) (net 10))
 (segment (start 108.585 81.915) (end 106.68 83.82) (width 0.25) (layer F.Cu) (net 13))
 (segment (start 111.825 81.915) (end 108.585 81.915) (width 0.25) (layer F.Cu) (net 13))
 (segment (start 116.775 79.375) (end 114.935 79.375) (width 0.25) (layer F.Cu) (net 12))
 (segment (start 114.935 79.375) (end 114.3 78.74) (width 0.25) (layer F.Cu) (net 12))
 (segment (start 114.3 71.12) (end 116.078 71.12) (width 0.25) (layer F.Cu) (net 1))
 (segment (start 116.775 71.817) (end 116.775 75.565) (width 0.25) (layer F.Cu) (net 1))
 (segment (start 116.078 71.12) (end 116.775 71.817) (width 0.25) (layer F.Cu) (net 1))
 (segment (start 110.871 74.549) (end 114.3 71.12) (width 1.5) (layer B.Cu) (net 1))
 (segment (start 110.871 78.985) (end 110.871 74.549) (width 1.5) (layer B.Cu) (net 1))
 (segment (start 111.825 84.455) (end 110.109 84.455) (width 0.25) (layer F.Cu) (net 2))
 (segment (start 110.109 84.455) (end 109.474 85.09) (width 0.25) (layer F.Cu) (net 2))
 (segment (start 109.474 86.106) (end 106.68 88.9) (width 0.25) (layer F.Cu) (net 2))
 (segment (start 109.474 85.09) (end 109.474 86.106) (width 0.25) (layer F.Cu) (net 2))
 (segment (start 110.871 84.709) (end 110.871 81.035) (width 1.5) (layer B.Cu) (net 2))
 (segment (start 106.68 88.9) (end 110.871 84.709) (width 1.5) (layer B.Cu) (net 2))
 (via (at 110.617 71.882) (size 0.8) (drill 0.4) (layers F.Cu B.Cu) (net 2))
 (via (at 108.458 73.787) (size 0.8) (drill 0.4) (layers F.Cu B.Cu) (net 2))
 (via (at 108.458 76.708) (size 0.8) (drill 0.4) (layers F.Cu B.Cu) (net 2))
 (via (at 108.458 80.01) (size 0.8) (drill 0.4) (layers F.Cu B.Cu) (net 2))
 (via (at 108.458 83.312) (size 0.8) (drill 0.4) (layers F.Cu B.Cu) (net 2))
 (via (at 110.998 88.011) (size 0.8) (drill 0.4) (layers F.Cu B.Cu) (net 2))
 (via (at 117.094 89.154) (size 0.8) (drill 0.4) (layers F.Cu B.Cu) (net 2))
 (via (at 117.094 70.866) (size 0.8) (drill 0.4) (layers F.Cu B.Cu) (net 2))
 (segment (start 114.56563 77.597) (end 114.3 77.33137) (width 0.25) (layer F.Cu) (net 14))
 (segment (start 114.3 77.33137) (end 114.3 76.2) (width 0.25) (layer F.Cu) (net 14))
 (segment (start 115.062 77.597) (end 114.56563 77.597) (width 0.25) (layer F.Cu) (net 14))
 (segment (start 115.57 78.105) (end 115.062 77.597) (width 0.25) (layer F.Cu) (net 14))
 (segment (start 116.775 78.105) (end 115.57 78.105) (width 0.25) (layer F.Cu) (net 14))
 (segment (start 109.855 83.185) (end 106.68 86.36) (width 0.25) (layer F.Cu) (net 15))
 (segment (start 111.825 83.185) (end 109.855 83.185) (width 0.25) (layer F.Cu) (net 15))
 (segment (start 115.099999 74.459999) (end 114.3 73.66) (width 0.25) (layer F.Cu) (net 16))
 (segment (start 115.425001 74.785001) (end 115.099999 74.459999) (width 0.25) (layer F.Cu) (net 16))
 (segment (start 115.425001 75.861769) (end 115.425001 74.785001) (width 0.25) (layer F.Cu) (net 16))
 (segment (start 115.753242 76.19001) (end 115.425001 75.861769) (width 0.25) (layer F.Cu) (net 16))
 (segment (start 116.13001 76.19001) (end 115.753242 76.19001) (width 0.25) (layer F.Cu) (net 16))
 (segment (start 116.775 76.835) (end 116.13001 76.19001) (width 0.25) (layer F.Cu) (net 16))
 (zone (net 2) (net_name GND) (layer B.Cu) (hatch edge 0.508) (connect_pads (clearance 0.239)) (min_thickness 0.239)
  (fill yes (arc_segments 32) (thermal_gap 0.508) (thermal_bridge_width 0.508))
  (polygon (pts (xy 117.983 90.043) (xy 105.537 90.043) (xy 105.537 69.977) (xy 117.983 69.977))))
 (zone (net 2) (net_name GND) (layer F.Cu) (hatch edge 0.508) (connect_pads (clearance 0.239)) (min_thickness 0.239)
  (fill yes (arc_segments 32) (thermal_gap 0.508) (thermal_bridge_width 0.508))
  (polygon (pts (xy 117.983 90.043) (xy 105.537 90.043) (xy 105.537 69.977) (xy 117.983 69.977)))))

